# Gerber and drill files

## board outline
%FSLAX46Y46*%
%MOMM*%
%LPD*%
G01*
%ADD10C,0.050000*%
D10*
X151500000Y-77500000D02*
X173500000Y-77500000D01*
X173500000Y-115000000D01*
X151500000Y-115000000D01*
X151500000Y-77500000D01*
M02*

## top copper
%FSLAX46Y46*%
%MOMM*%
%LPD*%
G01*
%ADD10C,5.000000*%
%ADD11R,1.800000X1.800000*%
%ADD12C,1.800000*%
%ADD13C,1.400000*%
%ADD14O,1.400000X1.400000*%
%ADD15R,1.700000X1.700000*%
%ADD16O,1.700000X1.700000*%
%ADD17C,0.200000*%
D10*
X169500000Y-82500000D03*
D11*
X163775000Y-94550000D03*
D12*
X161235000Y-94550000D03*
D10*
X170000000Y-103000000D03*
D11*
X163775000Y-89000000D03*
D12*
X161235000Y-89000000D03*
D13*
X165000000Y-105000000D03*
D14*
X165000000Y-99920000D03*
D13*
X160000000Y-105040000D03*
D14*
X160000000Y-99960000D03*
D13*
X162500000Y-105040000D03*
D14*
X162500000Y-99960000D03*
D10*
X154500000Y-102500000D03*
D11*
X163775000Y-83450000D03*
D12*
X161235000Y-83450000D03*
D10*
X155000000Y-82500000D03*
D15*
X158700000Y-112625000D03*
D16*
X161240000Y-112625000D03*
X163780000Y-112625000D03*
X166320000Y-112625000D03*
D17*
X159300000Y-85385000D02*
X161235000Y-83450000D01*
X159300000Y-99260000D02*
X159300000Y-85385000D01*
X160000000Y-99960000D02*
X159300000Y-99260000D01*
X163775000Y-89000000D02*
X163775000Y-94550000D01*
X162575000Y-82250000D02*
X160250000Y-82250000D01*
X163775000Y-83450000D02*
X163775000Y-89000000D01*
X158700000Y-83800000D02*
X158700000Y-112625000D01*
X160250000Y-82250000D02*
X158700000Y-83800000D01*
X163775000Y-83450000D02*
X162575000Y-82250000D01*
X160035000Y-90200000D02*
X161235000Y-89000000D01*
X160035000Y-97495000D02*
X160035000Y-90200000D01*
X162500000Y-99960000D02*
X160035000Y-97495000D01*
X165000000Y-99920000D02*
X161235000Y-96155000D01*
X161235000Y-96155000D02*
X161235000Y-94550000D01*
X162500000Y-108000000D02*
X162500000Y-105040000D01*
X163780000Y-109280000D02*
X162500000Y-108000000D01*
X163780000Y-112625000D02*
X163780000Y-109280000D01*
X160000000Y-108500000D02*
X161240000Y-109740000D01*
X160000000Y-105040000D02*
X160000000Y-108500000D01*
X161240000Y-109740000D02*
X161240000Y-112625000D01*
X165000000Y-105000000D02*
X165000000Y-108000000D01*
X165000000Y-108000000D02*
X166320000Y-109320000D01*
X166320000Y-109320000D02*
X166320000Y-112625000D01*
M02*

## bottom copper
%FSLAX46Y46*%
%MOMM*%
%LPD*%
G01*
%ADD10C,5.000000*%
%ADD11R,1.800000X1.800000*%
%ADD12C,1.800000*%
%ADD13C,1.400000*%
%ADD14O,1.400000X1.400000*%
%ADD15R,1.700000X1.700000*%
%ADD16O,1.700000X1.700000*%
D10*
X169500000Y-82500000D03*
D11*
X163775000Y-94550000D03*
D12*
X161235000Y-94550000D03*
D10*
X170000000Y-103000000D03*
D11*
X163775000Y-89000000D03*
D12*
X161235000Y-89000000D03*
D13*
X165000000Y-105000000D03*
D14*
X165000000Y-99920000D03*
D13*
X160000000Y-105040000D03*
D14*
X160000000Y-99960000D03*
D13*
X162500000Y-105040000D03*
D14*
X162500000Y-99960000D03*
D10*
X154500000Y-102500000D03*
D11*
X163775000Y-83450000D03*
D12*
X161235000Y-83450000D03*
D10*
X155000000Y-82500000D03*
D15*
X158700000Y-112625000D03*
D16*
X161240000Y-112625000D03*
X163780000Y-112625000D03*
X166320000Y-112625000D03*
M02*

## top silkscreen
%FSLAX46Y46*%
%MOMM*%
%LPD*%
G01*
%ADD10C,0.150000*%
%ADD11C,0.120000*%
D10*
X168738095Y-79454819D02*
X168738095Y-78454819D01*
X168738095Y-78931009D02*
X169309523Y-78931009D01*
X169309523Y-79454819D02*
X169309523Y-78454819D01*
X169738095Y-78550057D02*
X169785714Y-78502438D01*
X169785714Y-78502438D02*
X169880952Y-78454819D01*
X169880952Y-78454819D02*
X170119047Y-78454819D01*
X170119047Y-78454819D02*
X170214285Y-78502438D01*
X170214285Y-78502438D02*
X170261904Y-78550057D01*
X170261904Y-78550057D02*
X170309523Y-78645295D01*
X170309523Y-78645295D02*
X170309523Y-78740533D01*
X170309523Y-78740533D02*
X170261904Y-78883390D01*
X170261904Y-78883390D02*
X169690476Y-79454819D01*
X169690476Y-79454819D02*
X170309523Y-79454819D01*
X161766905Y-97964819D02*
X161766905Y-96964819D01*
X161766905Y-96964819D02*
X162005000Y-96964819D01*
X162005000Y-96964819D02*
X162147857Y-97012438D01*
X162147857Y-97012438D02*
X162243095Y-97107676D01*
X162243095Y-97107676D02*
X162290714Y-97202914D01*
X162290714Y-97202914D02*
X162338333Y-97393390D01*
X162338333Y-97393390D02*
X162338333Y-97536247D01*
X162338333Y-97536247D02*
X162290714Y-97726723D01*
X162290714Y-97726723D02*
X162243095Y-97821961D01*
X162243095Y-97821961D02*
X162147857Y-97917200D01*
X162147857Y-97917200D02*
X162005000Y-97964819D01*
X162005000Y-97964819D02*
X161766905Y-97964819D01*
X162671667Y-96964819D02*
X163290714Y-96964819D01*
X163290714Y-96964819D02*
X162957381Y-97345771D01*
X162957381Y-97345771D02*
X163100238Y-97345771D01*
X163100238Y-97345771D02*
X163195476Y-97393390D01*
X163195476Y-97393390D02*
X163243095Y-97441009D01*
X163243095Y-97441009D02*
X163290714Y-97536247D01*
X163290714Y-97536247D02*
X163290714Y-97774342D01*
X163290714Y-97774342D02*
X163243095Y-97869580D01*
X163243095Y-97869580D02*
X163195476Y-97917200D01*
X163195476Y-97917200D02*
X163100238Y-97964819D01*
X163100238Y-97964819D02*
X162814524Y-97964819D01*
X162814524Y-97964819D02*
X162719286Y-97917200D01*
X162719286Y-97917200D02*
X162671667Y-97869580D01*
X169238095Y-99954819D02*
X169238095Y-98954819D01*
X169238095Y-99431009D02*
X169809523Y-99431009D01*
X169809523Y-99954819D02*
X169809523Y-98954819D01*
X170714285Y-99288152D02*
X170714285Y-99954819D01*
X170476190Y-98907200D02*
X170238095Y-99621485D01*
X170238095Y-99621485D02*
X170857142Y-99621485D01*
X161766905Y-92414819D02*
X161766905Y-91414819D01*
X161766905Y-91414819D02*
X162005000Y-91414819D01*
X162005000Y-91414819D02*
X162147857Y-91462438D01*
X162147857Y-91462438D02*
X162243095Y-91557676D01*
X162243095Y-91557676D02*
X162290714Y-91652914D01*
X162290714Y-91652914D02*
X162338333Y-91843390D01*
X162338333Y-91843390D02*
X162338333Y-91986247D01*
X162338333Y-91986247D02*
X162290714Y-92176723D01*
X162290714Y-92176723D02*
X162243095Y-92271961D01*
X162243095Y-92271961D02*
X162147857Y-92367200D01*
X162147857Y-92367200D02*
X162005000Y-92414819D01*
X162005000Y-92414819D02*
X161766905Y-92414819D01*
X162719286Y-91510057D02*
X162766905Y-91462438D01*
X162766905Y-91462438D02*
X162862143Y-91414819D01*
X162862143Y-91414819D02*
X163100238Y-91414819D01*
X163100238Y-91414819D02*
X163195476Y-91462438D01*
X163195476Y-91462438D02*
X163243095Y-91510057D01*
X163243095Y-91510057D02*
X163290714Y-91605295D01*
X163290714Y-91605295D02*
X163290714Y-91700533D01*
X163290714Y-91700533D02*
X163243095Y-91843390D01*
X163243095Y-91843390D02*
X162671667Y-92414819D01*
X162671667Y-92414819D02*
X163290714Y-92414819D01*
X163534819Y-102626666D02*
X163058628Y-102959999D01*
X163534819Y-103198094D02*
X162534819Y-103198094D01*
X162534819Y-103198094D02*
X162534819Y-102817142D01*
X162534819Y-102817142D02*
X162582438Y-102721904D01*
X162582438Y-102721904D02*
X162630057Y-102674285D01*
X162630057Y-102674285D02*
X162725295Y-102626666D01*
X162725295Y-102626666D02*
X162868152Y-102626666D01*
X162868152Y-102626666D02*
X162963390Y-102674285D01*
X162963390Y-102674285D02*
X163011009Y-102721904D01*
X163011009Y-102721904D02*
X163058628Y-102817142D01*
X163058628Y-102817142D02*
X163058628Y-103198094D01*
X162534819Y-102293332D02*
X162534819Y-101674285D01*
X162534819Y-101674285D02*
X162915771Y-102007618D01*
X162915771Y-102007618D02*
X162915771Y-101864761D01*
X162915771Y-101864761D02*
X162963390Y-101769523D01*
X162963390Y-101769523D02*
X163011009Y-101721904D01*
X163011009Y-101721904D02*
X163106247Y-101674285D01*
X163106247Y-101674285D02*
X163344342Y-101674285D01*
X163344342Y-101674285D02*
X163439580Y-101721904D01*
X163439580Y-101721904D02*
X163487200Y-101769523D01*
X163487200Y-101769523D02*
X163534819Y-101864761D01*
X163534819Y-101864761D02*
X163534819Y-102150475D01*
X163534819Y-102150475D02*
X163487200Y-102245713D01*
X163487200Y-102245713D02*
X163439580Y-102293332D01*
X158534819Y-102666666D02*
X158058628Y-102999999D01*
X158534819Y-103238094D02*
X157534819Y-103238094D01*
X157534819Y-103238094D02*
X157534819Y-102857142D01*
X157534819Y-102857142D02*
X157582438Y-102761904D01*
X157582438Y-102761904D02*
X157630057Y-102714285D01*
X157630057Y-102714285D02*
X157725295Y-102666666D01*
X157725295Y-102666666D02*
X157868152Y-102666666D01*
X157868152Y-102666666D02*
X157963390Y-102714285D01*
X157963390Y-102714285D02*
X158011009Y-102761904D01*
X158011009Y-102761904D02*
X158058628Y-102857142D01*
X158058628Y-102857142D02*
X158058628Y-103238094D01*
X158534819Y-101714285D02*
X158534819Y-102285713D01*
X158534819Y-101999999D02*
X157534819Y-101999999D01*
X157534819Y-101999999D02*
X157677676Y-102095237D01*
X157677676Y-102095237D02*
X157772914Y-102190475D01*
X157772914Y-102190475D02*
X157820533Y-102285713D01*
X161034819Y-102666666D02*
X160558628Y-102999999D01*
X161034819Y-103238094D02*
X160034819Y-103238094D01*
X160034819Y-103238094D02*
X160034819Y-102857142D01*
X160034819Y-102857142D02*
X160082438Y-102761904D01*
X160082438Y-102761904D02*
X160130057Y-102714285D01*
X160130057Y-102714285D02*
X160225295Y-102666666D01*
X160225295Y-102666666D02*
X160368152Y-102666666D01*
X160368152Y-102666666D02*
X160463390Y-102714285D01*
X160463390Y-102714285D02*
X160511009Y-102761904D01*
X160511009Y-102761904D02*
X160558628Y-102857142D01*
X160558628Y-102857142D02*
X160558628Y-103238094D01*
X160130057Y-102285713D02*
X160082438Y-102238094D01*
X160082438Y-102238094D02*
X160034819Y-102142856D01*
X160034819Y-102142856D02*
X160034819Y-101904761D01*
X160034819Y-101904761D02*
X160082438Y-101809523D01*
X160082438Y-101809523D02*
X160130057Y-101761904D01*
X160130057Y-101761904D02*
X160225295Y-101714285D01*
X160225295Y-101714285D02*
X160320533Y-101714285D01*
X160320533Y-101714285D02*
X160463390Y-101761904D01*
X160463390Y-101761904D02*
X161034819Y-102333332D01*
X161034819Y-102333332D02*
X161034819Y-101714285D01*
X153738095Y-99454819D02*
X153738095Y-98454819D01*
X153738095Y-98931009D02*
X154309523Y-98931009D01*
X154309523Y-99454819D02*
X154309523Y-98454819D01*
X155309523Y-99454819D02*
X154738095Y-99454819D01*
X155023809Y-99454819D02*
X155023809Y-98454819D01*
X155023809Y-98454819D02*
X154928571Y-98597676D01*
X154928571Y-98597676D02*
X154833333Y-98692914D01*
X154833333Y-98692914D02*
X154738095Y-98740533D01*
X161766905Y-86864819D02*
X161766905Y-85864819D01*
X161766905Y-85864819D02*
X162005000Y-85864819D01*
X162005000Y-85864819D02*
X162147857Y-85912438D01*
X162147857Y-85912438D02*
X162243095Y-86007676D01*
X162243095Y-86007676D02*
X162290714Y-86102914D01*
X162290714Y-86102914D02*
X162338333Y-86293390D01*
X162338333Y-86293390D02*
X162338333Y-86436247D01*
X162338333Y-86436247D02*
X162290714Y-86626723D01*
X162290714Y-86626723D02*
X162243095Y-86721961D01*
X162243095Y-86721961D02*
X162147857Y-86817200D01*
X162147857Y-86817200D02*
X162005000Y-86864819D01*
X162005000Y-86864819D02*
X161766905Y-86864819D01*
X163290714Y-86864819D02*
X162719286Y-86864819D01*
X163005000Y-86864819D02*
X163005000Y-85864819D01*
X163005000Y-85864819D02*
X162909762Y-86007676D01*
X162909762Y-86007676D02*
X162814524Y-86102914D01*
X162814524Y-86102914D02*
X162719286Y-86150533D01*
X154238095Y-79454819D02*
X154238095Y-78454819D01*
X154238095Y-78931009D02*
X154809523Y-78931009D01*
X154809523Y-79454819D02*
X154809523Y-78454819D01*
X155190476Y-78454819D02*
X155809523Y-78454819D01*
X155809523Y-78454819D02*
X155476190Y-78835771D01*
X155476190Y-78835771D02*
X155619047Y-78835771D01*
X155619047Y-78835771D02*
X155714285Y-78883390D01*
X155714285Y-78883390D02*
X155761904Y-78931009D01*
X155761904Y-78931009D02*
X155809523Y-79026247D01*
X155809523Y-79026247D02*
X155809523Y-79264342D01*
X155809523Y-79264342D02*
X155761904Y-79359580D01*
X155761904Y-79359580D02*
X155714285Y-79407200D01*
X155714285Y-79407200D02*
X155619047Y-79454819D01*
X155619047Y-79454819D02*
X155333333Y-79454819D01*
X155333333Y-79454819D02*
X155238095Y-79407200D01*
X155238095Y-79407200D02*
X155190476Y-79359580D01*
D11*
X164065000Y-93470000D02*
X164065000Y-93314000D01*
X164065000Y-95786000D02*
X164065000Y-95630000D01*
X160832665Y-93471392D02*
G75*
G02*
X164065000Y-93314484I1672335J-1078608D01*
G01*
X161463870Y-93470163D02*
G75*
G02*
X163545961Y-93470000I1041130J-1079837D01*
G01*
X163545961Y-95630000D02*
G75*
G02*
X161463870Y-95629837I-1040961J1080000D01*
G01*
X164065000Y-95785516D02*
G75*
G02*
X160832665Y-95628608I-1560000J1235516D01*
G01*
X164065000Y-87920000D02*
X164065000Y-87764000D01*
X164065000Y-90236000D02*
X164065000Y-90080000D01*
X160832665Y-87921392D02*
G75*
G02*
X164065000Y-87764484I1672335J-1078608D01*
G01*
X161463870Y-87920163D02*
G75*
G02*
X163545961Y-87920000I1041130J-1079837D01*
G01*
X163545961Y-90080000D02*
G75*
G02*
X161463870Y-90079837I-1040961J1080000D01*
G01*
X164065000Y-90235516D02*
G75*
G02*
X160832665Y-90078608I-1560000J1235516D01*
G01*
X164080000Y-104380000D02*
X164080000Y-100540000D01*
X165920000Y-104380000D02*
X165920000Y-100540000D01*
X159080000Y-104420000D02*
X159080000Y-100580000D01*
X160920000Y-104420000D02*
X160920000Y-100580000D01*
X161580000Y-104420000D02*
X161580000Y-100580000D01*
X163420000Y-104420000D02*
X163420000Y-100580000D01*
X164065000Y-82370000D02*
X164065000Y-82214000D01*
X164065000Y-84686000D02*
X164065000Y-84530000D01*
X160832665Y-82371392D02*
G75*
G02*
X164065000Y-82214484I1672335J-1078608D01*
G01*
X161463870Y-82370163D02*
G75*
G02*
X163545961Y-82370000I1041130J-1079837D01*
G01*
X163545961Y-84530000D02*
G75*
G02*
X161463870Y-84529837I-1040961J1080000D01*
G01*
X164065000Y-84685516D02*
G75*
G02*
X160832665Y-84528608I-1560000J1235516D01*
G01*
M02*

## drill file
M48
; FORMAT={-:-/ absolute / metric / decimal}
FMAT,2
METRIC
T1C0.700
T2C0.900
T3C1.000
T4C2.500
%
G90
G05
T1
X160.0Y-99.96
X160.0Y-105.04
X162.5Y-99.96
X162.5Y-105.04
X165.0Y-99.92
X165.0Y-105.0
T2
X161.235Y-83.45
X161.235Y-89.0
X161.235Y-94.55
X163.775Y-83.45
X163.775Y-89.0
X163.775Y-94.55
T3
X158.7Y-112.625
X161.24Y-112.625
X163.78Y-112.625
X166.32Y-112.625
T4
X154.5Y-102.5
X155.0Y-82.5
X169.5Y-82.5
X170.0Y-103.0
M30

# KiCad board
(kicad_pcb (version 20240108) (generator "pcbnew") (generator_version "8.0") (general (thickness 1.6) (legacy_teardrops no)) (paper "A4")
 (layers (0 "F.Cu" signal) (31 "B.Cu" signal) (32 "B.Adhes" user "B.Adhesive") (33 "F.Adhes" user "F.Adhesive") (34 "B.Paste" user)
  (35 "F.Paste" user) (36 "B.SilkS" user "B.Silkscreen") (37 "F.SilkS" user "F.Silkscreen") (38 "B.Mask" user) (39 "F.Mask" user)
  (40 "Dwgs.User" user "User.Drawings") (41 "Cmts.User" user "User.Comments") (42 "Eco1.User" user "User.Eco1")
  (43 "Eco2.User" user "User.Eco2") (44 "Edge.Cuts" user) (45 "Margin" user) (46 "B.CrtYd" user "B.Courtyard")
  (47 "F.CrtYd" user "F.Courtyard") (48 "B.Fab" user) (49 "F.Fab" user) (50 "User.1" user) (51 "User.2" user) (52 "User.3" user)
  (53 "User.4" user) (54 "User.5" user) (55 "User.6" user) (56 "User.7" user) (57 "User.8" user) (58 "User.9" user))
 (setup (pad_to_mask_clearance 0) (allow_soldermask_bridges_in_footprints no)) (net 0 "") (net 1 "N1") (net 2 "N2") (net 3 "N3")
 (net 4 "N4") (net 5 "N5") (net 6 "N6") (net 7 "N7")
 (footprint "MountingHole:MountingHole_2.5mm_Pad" (layer "F.Cu") (at 169.5 82.5)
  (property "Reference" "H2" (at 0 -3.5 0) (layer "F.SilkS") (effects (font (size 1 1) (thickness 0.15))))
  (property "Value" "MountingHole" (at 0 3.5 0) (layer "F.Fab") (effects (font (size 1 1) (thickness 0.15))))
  (pad "1" thru_hole circle (at 0 0) (size 5 5) (drill 2.5) (layers "*.Cu" "*.Mask") (remove_unused_layers no)))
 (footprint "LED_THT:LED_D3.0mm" (layer "F.Cu") (at 163.775 94.55 180)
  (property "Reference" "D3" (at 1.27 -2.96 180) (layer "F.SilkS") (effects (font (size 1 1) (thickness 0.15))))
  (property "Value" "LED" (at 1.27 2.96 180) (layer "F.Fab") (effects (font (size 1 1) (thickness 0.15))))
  (fp_line (start -0.29 1.08) (end -0.29 1.236) (stroke (width 0.12) (type solid)) (layer "F.SilkS"))
  (fp_line (start -0.29 -1.236) (end -0.29 -1.08) (stroke (width 0.12) (type solid)) (layer "F.SilkS"))
  (fp_arc (start 2.942335 1.078608) (mid 1.366487 1.987659) (end -0.29 1.235516) (stroke (width 0.12) (type solid)) (layer "F.SilkS"))
  (fp_arc (start 2.31113 1.079837) (mid 1.270117 1.5) (end 0.229039 1.08) (stroke (width 0.12) (type solid)) (layer "F.SilkS"))
  (fp_arc (start 0.229039 -1.08) (mid 1.270117 -1.5) (end 2.31113 -1.079837) (stroke (width 0.12) (type solid)) (layer "F.SilkS"))
  (fp_arc (start -0.29 -1.235516) (mid 1.366487 -1.987659) (end 2.942335 -1.078608) (stroke (width 0.12) (type solid)) (layer "F.SilkS"))
  (pad "1" thru_hole rect (at 0 0 180) (size 1.8 1.8) (drill 0.9) (layers "*.Cu" "*.Mask") (remove_unused_layers no) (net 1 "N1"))
  (pad "2" thru_hole circle (at 2.54 0 180) (size 1.8 1.8) (drill 0.9) (layers "*.Cu" "*.Mask") (remove_unused_layers no) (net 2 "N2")))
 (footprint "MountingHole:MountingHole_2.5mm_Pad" (layer "F.Cu") (at 170 103)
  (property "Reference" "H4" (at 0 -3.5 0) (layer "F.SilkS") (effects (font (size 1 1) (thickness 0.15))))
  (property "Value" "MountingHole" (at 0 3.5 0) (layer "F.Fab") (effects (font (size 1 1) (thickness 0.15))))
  (pad "1" thru_hole circle (at 0 0) (size 5 5) (drill 2.5) (layers "*.Cu" "*.Mask") (remove_unused_layers no)))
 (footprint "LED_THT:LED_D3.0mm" (layer "F.Cu") (at 163.775 89 180)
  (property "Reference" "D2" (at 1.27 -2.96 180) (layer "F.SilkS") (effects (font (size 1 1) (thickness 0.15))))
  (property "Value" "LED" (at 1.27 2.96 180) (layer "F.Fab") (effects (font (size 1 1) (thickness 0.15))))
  (fp_line (start -0.29 1.08) (end -0.29 1.236) (stroke (width 0.12) (type solid)) (layer "F.SilkS"))
  (fp_line (start -0.29 -1.236) (end -0.29 -1.08) (stroke (width 0.12) (type solid)) (layer "F.SilkS"))
  (fp_arc (start 2.942335 1.078608) (mid 1.366487 1.987659) (end -0.29 1.235516) (stroke (width 0.12) (type solid)) (layer "F.SilkS"))
  (fp_arc (start 2.31113 1.079837) (mid 1.270117 1.5) (end 0.229039 1.08) (stroke (width 0.12) (type solid)) (layer "F.SilkS"))
  (fp_arc (start 0.229039 -1.08) (mid 1.270117 -1.5) (end 2.31113 -1.079837) (stroke (width 0.12) (type solid)) (layer "F.SilkS"))
  (fp_arc (start -0.29 -1.235516) (mid 1.366487 -1.987659) (end 2.942335 -1.078608) (stroke (width 0.12) (type solid)) (layer "F.SilkS"))
  (pad "1" thru_hole rect (at 0 0 180) (size 1.8 1.8) (drill 0.9) (layers "*.Cu" "*.Mask") (remove_unused_layers no) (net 1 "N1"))
  (pad "2" thru_hole circle (at 2.54 0 180) (size 1.8 1.8) (drill 0.9) (layers "*.Cu" "*.Mask") (remove_unused_layers no) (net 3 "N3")))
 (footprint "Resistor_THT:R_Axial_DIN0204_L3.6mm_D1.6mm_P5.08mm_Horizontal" (layer "F.Cu") (at 165 105 90)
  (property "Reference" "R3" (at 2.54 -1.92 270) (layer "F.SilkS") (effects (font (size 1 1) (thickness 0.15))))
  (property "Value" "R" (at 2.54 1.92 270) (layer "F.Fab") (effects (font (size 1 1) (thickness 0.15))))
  (fp_line (start 0.62 -0.92) (end 4.46 -0.92) (stroke (width 0.12) (type solid)) (layer "F.SilkS"))
  (fp_line (start 0.62 0.92) (end 4.46 0.92) (stroke (width 0.12) (type solid)) (layer "F.SilkS"))
  (pad "1" thru_hole circle (at 0 0 90) (size 1.4 1.4) (drill 0.7) (layers "*.Cu" "*.Mask") (remove_unused_layers no) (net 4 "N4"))
  (pad "2" thru_hole oval (at 5.08 0 90) (size 1.4 1.4) (drill 0.7) (layers "*.Cu" "*.Mask") (remove_unused_layers no) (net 2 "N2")))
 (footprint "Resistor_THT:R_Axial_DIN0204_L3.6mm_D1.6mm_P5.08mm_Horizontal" (layer "F.Cu") (at 160 105.04 90)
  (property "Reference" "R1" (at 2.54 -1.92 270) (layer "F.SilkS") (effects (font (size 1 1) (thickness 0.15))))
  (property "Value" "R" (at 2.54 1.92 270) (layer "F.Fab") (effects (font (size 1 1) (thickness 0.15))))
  (fp_line (start 0.62 -0.92) (end 4.46 -0.92) (stroke (width 0.12) (type solid)) (layer "F.SilkS"))
  (fp_line (start 0.62 0.92) (end 4.46 0.92) (stroke (width 0.12) (type solid)) (layer "F.SilkS"))
  (pad "1" thru_hole circle (at 0 0 90) (size 1.4 1.4) (drill 0.7) (layers "*.Cu" "*.Mask") (remove_unused_layers no) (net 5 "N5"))
  (pad "2" thru_hole oval (at 5.08 0 90) (size 1.4 1.4) (drill 0.7) (layers "*.Cu" "*.Mask") (remove_unused_layers no) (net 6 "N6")))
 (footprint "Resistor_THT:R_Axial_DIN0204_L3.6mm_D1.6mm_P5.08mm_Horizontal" (layer "F.Cu") (at 162.5 105.04 90)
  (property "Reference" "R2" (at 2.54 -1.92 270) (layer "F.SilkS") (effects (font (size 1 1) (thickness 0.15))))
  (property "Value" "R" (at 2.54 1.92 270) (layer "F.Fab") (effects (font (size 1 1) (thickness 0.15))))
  (fp_line (start 0.62 -0.92) (end 4.46 -0.92) (stroke (width 0.12) (type solid)) (layer "F.SilkS"))
  (fp_line (start 0.62 0.92) (end 4.46 0.92) (stroke (width 0.12) (type solid)) (layer "F.SilkS"))
  (pad "1" thru_hole circle (at 0 0 90) (size 1.4 1.4) (drill 0.7) (layers "*.Cu" "*.Mask") (remove_unused_layers no) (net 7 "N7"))
  (pad "2" thru_hole oval (at 5.08 0 90) (size 1.4 1.4) (drill 0.7) (layers "*.Cu" "*.Mask") (remove_unused_layers no) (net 3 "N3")))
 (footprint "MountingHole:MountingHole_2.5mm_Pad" (layer "F.Cu") (at 154.5 102.5)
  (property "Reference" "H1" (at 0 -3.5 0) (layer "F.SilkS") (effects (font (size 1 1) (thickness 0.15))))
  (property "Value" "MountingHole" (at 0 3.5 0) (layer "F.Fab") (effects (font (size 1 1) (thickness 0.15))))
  (pad "1" thru_hole circle (at 0 0) (size 5 5) (drill 2.5) (layers "*.Cu" "*.Mask") (remove_unused_layers no)))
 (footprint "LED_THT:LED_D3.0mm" (layer "F.Cu") (at 163.775 83.45 180)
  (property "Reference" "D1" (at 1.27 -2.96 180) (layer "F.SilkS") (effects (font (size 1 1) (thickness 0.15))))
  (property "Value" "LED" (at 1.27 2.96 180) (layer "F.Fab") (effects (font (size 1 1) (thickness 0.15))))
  (fp_line (start -0.29 1.08) (end -0.29 1.236) (stroke (width 0.12) (type solid)) (layer "F.SilkS"))
  (fp_line (start -0.29 -1.236) (end -0.29 -1.08) (stroke (width 0.12) (type solid)) (layer "F.SilkS"))
  (fp_arc (start 2.942335 1.078608) (mid 1.366487 1.987659) (end -0.29 1.235516) (stroke (width 0.12) (type solid)) (layer "F.SilkS"))
  (fp_arc (start 2.31113 1.079837) (mid 1.270117 1.5) (end 0.229039 1.08) (stroke (width 0.12) (type solid)) (layer "F.SilkS"))
  (fp_arc (start 0.229039 -1.08) (mid 1.270117 -1.5) (end 2.31113 -1.079837) (stroke (width 0.12) (type solid)) (layer "F.SilkS"))
  (fp_arc (start -0.29 -1.235516) (mid 1.366487 -1.987659) (end 2.942335 -1.078608) (stroke (width 0.12) (type solid)) (layer "F.SilkS"))
  (pad "1" thru_hole rect (at 0 0 180) (size 1.8 1.8) (drill 0.9) (layers "*.Cu" "*.Mask") (remove_unused_layers no) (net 1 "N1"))
  (pad "2" thru_hole circle (at 2.54 0 180) (size 1.8 1.8) (drill 0.9) (layers "*.Cu" "*.Mask") (remove_unused_layers no) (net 6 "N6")))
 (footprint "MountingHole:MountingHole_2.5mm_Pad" (layer "F.Cu") (at 155 82.5)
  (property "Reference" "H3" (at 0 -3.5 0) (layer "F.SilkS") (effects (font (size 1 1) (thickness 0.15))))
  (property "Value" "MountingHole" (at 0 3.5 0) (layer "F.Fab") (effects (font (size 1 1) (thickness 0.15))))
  (pad "1" thru_hole circle (at 0 0) (size 5 5) (drill 2.5) (layers "*.Cu" "*.Mask") (remove_unused_layers no)))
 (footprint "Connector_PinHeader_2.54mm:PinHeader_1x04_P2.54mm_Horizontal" (layer "B.Cu") (at 158.7 112.625 -90)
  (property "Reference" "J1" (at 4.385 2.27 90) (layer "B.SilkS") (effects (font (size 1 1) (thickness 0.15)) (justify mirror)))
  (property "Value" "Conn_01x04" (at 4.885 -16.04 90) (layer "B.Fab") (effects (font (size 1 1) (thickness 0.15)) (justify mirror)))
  (pad "1" thru_hole rect (at 0 0 270) (size 1.7 1.7) (drill 1) (layers "*.Cu" "*.Mask") (remove_unused_layers no) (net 1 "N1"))
  (pad "2" thru_hole oval (at 0 -2.54 270) (size 1.7 1.7) (drill 1) (layers "*.Cu" "*.Mask") (remove_unused_layers no) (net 5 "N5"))
  (pad "3" thru_hole oval (at 0 -5.08 270) (size 1.7 1.7) (drill 1) (layers "*.Cu" "*.Mask") (remove_unused_layers no) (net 7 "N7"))
  (pad "4" thru_hole oval (at 0 -7.62 270) (size 1.7 1.7) (drill 1) (layers "*.Cu" "*.Mask") (remove_unused_layers no) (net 4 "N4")))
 (gr_rect (start 151.5 77.5) (end 173.5 115) (stroke (width 0.05) (type default)) (fill none) (layer "Edge.Cuts"))
 (segment (start 159.3 85.385) (end 161.235 83.45) (width 0.2) (layer "F.Cu") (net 6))
 (segment (start 159.3 99.26) (end 159.3 85.385) (width 0.2) (layer "F.Cu") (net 6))
 (segment (start 160 99.96) (end 159.3 99.26) (width 0.2) (layer "F.Cu") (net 6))
 (segment (start 163.775 89) (end 163.775 94.55) (width 0.2) (layer "F.Cu") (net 1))
 (segment (start 162.575 82.25) (end 160.25 82.25) (width 0.2) (layer "F.Cu") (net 1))
 (segment (start 163.775 83.45) (end 163.775 89) (width 0.2) (layer "F.Cu") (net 1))
 (segment (start 158.7 83.8) (end 158.7 112.625) (width 0.2) (layer "F.Cu") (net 1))
 (segment (start 160.25 82.25) (end 158.7 83.8) (width 0.2) (layer "F.Cu") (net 1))
 (segment (start 163.775 83.45) (end 162.575 82.25) (width 0.2) (layer "F.Cu") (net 1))
 (segment (start 160.035 90.2) (end 161.235 89) (width 0.2) (layer "F.Cu") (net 3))
 (segment (start 160.035 97.495) (end 160.035 90.2) (width 0.2) (layer "F.Cu") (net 3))
 (segment (start 162.5 99.96) (end 160.035 97.495) (width 0.2) (layer "F.Cu") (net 3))
 (segment (start 165 99.92) (end 161.235 96.155) (width 0.2) (layer "F.Cu") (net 2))
 (segment (start 161.235 96.155) (end 161.235 94.55) (width 0.2) (layer "F.Cu") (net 2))
 (segment (start 162.5 108) (end 162.5 105.04) (width 0.2) (layer "F.Cu") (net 7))
 (segment (start 163.78 109.28) (end 162.5 108) (width 0.2) (layer "F.Cu") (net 7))
 (segment (start 163.78 112.625) (end 163.78 109.28) (width 0.2) (layer "F.Cu") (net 7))
 (segment (start 160 108.5) (end 161.24 109.74) (width 0.2) (layer "F.Cu") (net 5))
 (segment (start 160 105.04) (end 160 108.5) (width 0.2) (layer "F.Cu") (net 5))
 (segment (start 161.24 109.74) (end 161.24 112.625) (width 0.2) (layer "F.Cu") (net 5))
 (segment (start 165 105) (end 165 108) (width 0.2) (layer "F.Cu") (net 4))
 (segment (start 165 108) (end 166.32 109.32) (width 0.2) (layer "F.Cu") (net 4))
 (segment (start 166.32 109.32) (end 166.32 112.625) (width 0.2) (layer "F.Cu") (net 4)))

